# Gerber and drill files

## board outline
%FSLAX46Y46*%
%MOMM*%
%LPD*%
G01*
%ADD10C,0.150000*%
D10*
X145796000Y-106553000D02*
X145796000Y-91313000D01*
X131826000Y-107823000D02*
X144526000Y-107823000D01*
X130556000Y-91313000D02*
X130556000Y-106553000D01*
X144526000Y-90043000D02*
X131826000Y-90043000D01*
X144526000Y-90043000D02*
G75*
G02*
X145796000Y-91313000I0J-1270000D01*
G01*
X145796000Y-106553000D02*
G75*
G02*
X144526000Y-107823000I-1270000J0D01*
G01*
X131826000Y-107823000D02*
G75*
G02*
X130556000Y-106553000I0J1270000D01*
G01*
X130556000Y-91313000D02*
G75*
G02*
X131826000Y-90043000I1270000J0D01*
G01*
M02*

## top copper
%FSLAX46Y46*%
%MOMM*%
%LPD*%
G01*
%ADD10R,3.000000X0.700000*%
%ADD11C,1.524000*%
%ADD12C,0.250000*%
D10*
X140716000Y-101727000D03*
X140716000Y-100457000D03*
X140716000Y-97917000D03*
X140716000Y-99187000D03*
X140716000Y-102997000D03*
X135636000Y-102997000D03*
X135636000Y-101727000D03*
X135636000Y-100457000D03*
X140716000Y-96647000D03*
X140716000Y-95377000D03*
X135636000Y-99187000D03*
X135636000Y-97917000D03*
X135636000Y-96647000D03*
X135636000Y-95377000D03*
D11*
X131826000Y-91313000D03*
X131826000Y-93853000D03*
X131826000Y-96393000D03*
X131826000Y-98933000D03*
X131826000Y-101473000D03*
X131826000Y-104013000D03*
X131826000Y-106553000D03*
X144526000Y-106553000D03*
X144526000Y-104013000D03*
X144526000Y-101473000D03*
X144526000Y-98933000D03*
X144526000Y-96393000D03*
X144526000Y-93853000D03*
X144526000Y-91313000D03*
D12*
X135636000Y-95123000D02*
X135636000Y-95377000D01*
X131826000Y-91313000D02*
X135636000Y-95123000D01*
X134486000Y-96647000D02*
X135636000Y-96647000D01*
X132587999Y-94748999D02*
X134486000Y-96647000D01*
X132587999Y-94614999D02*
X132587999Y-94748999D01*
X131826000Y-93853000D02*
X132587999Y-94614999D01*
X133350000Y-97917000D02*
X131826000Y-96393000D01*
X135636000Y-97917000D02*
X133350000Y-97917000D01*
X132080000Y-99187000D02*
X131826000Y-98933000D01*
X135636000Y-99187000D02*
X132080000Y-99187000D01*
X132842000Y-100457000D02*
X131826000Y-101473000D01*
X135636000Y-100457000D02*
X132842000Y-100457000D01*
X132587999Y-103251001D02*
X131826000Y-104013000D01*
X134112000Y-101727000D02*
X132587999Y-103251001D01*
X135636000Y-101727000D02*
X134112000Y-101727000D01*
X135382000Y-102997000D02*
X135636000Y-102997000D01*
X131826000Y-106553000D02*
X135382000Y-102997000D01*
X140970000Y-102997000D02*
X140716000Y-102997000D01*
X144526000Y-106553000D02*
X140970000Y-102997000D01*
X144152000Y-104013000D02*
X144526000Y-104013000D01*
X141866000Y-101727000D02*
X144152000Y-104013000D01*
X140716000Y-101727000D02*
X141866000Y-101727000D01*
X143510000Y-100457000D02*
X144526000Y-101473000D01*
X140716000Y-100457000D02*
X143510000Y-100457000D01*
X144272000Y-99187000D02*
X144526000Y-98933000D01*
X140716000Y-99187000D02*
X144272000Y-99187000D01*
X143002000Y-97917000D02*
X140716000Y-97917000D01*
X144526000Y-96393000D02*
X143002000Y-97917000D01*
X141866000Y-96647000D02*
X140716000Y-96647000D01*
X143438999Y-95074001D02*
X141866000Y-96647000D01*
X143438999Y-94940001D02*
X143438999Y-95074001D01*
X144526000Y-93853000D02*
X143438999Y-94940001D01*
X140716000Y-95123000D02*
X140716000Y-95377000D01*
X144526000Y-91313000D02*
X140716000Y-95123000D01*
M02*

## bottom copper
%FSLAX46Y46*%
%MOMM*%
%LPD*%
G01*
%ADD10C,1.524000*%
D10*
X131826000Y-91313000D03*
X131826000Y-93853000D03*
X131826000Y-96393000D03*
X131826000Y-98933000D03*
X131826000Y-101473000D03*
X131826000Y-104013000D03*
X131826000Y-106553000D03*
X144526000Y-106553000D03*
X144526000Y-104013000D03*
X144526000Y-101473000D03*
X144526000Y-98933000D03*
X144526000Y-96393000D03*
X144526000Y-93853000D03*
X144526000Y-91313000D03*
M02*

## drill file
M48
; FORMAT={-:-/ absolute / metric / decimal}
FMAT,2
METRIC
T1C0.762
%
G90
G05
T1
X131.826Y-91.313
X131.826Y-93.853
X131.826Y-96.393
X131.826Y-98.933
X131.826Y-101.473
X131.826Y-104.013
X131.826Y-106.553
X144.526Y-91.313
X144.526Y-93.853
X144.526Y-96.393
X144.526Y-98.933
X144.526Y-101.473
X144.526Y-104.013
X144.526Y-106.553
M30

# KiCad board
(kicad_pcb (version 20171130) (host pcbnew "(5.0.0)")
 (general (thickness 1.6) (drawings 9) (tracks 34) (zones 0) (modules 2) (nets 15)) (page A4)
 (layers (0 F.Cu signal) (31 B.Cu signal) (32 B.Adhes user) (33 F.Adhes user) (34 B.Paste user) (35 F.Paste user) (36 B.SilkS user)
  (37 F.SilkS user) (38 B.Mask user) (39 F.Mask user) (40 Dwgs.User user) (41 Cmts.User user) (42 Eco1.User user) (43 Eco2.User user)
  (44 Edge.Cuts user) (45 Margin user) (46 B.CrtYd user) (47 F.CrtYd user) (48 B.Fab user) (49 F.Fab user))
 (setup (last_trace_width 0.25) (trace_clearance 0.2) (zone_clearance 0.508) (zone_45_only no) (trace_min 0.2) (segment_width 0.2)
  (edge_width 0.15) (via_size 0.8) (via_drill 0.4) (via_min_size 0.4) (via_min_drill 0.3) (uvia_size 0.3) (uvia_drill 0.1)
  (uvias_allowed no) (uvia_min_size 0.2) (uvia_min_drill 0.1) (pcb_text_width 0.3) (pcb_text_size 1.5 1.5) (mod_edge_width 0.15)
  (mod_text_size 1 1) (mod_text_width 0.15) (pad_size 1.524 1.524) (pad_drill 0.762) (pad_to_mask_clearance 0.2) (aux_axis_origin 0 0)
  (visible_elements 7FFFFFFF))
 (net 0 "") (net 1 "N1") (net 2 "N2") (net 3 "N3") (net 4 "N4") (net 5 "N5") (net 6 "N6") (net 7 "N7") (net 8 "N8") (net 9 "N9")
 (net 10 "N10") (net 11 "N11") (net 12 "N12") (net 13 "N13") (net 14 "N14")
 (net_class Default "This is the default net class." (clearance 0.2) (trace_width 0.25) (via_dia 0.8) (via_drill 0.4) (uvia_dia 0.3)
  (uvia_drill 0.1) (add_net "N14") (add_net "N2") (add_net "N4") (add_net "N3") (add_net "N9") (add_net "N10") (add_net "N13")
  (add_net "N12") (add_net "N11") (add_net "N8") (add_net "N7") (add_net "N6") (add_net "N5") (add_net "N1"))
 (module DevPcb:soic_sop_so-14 (layer F.Cu) (at 138.176 94.107)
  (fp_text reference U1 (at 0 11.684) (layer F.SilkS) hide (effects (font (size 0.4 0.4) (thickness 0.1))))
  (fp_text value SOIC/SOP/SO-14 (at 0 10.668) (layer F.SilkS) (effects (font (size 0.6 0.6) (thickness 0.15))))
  (pad 9 smd rect (at 2.54 7.62 90) (size 0.7 3) (layers F.Cu F.Paste F.Mask) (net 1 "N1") (solder_mask_margin 0.1))
  (pad 10 smd rect (at 2.54 6.35 90) (size 0.7 3) (layers F.Cu F.Paste F.Mask) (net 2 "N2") (solder_mask_margin 0.1))
  (pad 12 smd rect (at 2.54 3.81 90) (size 0.7 3) (layers F.Cu F.Paste F.Mask) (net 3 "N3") (solder_mask_margin 0.1))
  (pad 11 smd rect (at 2.54 5.08 90) (size 0.7 3) (layers F.Cu F.Paste F.Mask) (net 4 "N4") (solder_mask_margin 0.1))
  (pad 8 smd rect (at 2.54 8.89 90) (size 0.7 3) (layers F.Cu F.Paste F.Mask) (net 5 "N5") (solder_mask_margin 0.1))
  (pad 7 smd rect (at -2.54 8.89 90) (size 0.7 3) (layers F.Cu F.Paste F.Mask) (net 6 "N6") (solder_mask_margin 0.1))
  (pad 6 smd rect (at -2.54 7.62 90) (size 0.7 3) (layers F.Cu F.Paste F.Mask) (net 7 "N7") (solder_mask_margin 0.1))
  (pad 5 smd rect (at -2.54 6.35 90) (size 0.7 3) (layers F.Cu F.Paste F.Mask) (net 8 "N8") (solder_mask_margin 0.1))
  (pad 13 smd rect (at 2.54 2.54 90) (size 0.7 3) (layers F.Cu F.Paste F.Mask) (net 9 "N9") (solder_mask_margin 0.1))
  (pad 14 smd rect (at 2.54 1.27 90) (size 0.7 3) (layers F.Cu F.Paste F.Mask) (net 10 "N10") (solder_mask_margin 0.1))
  (pad 4 smd rect (at -2.54 5.08 90) (size 0.7 3) (layers F.Cu F.Paste F.Mask) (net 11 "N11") (solder_mask_margin 0.1))
  (pad 3 smd rect (at -2.54 3.81 90) (size 0.7 3) (layers F.Cu F.Paste F.Mask) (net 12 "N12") (solder_mask_margin 0.1))
  (pad 2 smd rect (at -2.54 2.54 90) (size 0.7 3) (layers F.Cu F.Paste F.Mask) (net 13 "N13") (solder_mask_margin 0.1))
  (pad 1 smd rect (at -2.54 1.27 90) (size 0.7 3) (layers F.Cu F.Paste F.Mask) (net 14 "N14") (solder_mask_margin 0.1)))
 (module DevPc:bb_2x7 (layer F.Cu) (at 131.826 91.313)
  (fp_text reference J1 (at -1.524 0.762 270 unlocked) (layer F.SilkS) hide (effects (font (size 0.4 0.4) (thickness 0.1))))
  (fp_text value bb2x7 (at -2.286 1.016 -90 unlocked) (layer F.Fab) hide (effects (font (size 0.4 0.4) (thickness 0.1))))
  (pad 1 thru_hole circle (at 0 0) (size 1.524 1.524) (drill 0.762) (layers *.Cu *.Mask) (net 14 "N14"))
  (pad 2 thru_hole circle (at 0 2.54) (size 1.524 1.524) (drill 0.762) (layers *.Cu *.Mask) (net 13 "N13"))
  (pad 3 thru_hole circle (at 0 5.08) (size 1.524 1.524) (drill 0.762) (layers *.Cu *.Mask) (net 12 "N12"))
  (pad 4 thru_hole circle (at 0 7.62) (size 1.524 1.524) (drill 0.762) (layers *.Cu *.Mask) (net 11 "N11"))
  (pad 5 thru_hole circle (at 0 10.16) (size 1.524 1.524) (drill 0.762) (layers *.Cu *.Mask) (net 8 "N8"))
  (pad 6 thru_hole circle (at 0 12.7) (size 1.524 1.524) (drill 0.762) (layers *.Cu *.Mask) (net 7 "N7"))
  (pad 7 thru_hole circle (at 0 15.24) (size 1.524 1.524) (drill 0.762) (layers *.Cu *.Mask) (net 6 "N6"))
  (pad 8 thru_hole circle (at 12.7 15.24) (size 1.524 1.524) (drill 0.762) (layers *.Cu *.Mask) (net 5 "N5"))
  (pad 9 thru_hole circle (at 12.7 12.7) (size 1.524 1.524) (drill 0.762) (layers *.Cu *.Mask) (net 1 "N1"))
  (pad 10 thru_hole circle (at 12.7 10.16) (size 1.524 1.524) (drill 0.762) (layers *.Cu *.Mask) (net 2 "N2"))
  (pad 11 thru_hole circle (at 12.7 7.62) (size 1.524 1.524) (drill 0.762) (layers *.Cu *.Mask) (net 4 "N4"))
  (pad 12 thru_hole circle (at 12.7 5.08) (size 1.524 1.524) (drill 0.762) (layers *.Cu *.Mask) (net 3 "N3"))
  (pad 13 thru_hole circle (at 12.7 2.54) (size 1.524 1.524) (drill 0.762) (layers *.Cu *.Mask) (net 9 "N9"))
  (pad 14 thru_hole circle (at 12.7 0) (size 1.524 1.524) (drill 0.762) (layers *.Cu *.Mask) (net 10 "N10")))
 (gr_line (start 145.796 106.553) (end 145.796 91.313) (layer Edge.Cuts) (width 0.15))
 (gr_line (start 131.826 107.823) (end 144.526 107.823) (layer Edge.Cuts) (width 0.15))
 (gr_line (start 130.556 91.313) (end 130.556 106.553) (layer Edge.Cuts) (width 0.15))
 (gr_line (start 144.526 90.043) (end 131.826 90.043) (layer Edge.Cuts) (width 0.15))
 (gr_arc (start 144.526 91.313) (end 145.796 91.313) (angle -90) (layer Edge.Cuts) (width 0.15))
 (gr_arc (start 144.526 106.553) (end 144.526 107.823) (angle -90) (layer Edge.Cuts) (width 0.15))
 (gr_arc (start 131.826 106.553) (end 130.556 106.553) (angle -90) (layer Edge.Cuts) (width 0.15))
 (gr_arc (start 131.826 91.313) (end 131.826 90.043) (angle -90) (layer Edge.Cuts) (width 0.15))
 (segment (start 135.636 95.123) (end 135.636 95.377) (width 0.25) (layer F.Cu) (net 14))
 (segment (start 131.826 91.313) (end 135.636 95.123) (width 0.25) (layer F.Cu) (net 14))
 (segment (start 134.486 96.647) (end 135.636 96.647) (width 0.25) (layer F.Cu) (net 13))
 (segment (start 132.587999 94.748999) (end 134.486 96.647) (width 0.25) (layer F.Cu) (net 13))
 (segment (start 132.587999 94.614999) (end 132.587999 94.748999) (width 0.25) (layer F.Cu) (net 13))
 (segment (start 131.826 93.853) (end 132.587999 94.614999) (width 0.25) (layer F.Cu) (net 13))
 (segment (start 133.35 97.917) (end 131.826 96.393) (width 0.25) (layer F.Cu) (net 12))
 (segment (start 135.636 97.917) (end 133.35 97.917) (width 0.25) (layer F.Cu) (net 12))
 (segment (start 132.08 99.187) (end 131.826 98.933) (width 0.25) (layer F.Cu) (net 11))
 (segment (start 135.636 99.187) (end 132.08 99.187) (width 0.25) (layer F.Cu) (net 11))
 (segment (start 132.842 100.457) (end 131.826 101.473) (width 0.25) (layer F.Cu) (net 8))
 (segment (start 135.636 100.457) (end 132.842 100.457) (width 0.25) (layer F.Cu) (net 8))
 (segment (start 132.587999 103.251001) (end 131.826 104.013) (width 0.25) (layer F.Cu) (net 7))
 (segment (start 134.112 101.727) (end 132.587999 103.251001) (width 0.25) (layer F.Cu) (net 7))
 (segment (start 135.636 101.727) (end 134.112 101.727) (width 0.25) (layer F.Cu) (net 7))
 (segment (start 135.382 102.997) (end 135.636 102.997) (width 0.25) (layer F.Cu) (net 6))
 (segment (start 131.826 106.553) (end 135.382 102.997) (width 0.25) (layer F.Cu) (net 6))
 (segment (start 140.97 102.997) (end 140.716 102.997) (width 0.25) (layer F.Cu) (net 5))
 (segment (start 144.526 106.553) (end 140.97 102.997) (width 0.25) (layer F.Cu) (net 5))
 (segment (start 144.152 104.013) (end 144.526 104.013) (width 0.25) (layer F.Cu) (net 1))
 (segment (start 141.866 101.727) (end 144.152 104.013) (width 0.25) (layer F.Cu) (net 1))
 (segment (start 140.716 101.727) (end 141.866 101.727) (width 0.25) (layer F.Cu) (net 1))
 (segment (start 143.51 100.457) (end 144.526 101.473) (width 0.25) (layer F.Cu) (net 2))
 (segment (start 140.716 100.457) (end 143.51 100.457) (width 0.25) (layer F.Cu) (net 2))
 (segment (start 144.272 99.187) (end 144.526 98.933) (width 0.25) (layer F.Cu) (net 4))
 (segment (start 140.716 99.187) (end 144.272 99.187) (width 0.25) (layer F.Cu) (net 4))
 (segment (start 143.002 97.917) (end 140.716 97.917) (width 0.25) (layer F.Cu) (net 3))
 (segment (start 144.526 96.393) (end 143.002 97.917) (width 0.25) (layer F.Cu) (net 3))
 (segment (start 141.866 96.647) (end 140.716 96.647) (width 0.25) (layer F.Cu) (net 9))
 (segment (start 143.438999 95.074001) (end 141.866 96.647) (width 0.25) (layer F.Cu) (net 9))
 (segment (start 143.438999 94.940001) (end 143.438999 95.074001) (width 0.25) (layer F.Cu) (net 9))
 (segment (start 144.526 93.853) (end 143.438999 94.940001) (width 0.25) (layer F.Cu) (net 9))
 (segment (start 140.716 95.123) (end 140.716 95.377) (width 0.25) (layer F.Cu) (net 10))
 (segment (start 144.526 91.313) (end 140.716 95.123) (width 0.25) (layer F.Cu) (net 10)))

